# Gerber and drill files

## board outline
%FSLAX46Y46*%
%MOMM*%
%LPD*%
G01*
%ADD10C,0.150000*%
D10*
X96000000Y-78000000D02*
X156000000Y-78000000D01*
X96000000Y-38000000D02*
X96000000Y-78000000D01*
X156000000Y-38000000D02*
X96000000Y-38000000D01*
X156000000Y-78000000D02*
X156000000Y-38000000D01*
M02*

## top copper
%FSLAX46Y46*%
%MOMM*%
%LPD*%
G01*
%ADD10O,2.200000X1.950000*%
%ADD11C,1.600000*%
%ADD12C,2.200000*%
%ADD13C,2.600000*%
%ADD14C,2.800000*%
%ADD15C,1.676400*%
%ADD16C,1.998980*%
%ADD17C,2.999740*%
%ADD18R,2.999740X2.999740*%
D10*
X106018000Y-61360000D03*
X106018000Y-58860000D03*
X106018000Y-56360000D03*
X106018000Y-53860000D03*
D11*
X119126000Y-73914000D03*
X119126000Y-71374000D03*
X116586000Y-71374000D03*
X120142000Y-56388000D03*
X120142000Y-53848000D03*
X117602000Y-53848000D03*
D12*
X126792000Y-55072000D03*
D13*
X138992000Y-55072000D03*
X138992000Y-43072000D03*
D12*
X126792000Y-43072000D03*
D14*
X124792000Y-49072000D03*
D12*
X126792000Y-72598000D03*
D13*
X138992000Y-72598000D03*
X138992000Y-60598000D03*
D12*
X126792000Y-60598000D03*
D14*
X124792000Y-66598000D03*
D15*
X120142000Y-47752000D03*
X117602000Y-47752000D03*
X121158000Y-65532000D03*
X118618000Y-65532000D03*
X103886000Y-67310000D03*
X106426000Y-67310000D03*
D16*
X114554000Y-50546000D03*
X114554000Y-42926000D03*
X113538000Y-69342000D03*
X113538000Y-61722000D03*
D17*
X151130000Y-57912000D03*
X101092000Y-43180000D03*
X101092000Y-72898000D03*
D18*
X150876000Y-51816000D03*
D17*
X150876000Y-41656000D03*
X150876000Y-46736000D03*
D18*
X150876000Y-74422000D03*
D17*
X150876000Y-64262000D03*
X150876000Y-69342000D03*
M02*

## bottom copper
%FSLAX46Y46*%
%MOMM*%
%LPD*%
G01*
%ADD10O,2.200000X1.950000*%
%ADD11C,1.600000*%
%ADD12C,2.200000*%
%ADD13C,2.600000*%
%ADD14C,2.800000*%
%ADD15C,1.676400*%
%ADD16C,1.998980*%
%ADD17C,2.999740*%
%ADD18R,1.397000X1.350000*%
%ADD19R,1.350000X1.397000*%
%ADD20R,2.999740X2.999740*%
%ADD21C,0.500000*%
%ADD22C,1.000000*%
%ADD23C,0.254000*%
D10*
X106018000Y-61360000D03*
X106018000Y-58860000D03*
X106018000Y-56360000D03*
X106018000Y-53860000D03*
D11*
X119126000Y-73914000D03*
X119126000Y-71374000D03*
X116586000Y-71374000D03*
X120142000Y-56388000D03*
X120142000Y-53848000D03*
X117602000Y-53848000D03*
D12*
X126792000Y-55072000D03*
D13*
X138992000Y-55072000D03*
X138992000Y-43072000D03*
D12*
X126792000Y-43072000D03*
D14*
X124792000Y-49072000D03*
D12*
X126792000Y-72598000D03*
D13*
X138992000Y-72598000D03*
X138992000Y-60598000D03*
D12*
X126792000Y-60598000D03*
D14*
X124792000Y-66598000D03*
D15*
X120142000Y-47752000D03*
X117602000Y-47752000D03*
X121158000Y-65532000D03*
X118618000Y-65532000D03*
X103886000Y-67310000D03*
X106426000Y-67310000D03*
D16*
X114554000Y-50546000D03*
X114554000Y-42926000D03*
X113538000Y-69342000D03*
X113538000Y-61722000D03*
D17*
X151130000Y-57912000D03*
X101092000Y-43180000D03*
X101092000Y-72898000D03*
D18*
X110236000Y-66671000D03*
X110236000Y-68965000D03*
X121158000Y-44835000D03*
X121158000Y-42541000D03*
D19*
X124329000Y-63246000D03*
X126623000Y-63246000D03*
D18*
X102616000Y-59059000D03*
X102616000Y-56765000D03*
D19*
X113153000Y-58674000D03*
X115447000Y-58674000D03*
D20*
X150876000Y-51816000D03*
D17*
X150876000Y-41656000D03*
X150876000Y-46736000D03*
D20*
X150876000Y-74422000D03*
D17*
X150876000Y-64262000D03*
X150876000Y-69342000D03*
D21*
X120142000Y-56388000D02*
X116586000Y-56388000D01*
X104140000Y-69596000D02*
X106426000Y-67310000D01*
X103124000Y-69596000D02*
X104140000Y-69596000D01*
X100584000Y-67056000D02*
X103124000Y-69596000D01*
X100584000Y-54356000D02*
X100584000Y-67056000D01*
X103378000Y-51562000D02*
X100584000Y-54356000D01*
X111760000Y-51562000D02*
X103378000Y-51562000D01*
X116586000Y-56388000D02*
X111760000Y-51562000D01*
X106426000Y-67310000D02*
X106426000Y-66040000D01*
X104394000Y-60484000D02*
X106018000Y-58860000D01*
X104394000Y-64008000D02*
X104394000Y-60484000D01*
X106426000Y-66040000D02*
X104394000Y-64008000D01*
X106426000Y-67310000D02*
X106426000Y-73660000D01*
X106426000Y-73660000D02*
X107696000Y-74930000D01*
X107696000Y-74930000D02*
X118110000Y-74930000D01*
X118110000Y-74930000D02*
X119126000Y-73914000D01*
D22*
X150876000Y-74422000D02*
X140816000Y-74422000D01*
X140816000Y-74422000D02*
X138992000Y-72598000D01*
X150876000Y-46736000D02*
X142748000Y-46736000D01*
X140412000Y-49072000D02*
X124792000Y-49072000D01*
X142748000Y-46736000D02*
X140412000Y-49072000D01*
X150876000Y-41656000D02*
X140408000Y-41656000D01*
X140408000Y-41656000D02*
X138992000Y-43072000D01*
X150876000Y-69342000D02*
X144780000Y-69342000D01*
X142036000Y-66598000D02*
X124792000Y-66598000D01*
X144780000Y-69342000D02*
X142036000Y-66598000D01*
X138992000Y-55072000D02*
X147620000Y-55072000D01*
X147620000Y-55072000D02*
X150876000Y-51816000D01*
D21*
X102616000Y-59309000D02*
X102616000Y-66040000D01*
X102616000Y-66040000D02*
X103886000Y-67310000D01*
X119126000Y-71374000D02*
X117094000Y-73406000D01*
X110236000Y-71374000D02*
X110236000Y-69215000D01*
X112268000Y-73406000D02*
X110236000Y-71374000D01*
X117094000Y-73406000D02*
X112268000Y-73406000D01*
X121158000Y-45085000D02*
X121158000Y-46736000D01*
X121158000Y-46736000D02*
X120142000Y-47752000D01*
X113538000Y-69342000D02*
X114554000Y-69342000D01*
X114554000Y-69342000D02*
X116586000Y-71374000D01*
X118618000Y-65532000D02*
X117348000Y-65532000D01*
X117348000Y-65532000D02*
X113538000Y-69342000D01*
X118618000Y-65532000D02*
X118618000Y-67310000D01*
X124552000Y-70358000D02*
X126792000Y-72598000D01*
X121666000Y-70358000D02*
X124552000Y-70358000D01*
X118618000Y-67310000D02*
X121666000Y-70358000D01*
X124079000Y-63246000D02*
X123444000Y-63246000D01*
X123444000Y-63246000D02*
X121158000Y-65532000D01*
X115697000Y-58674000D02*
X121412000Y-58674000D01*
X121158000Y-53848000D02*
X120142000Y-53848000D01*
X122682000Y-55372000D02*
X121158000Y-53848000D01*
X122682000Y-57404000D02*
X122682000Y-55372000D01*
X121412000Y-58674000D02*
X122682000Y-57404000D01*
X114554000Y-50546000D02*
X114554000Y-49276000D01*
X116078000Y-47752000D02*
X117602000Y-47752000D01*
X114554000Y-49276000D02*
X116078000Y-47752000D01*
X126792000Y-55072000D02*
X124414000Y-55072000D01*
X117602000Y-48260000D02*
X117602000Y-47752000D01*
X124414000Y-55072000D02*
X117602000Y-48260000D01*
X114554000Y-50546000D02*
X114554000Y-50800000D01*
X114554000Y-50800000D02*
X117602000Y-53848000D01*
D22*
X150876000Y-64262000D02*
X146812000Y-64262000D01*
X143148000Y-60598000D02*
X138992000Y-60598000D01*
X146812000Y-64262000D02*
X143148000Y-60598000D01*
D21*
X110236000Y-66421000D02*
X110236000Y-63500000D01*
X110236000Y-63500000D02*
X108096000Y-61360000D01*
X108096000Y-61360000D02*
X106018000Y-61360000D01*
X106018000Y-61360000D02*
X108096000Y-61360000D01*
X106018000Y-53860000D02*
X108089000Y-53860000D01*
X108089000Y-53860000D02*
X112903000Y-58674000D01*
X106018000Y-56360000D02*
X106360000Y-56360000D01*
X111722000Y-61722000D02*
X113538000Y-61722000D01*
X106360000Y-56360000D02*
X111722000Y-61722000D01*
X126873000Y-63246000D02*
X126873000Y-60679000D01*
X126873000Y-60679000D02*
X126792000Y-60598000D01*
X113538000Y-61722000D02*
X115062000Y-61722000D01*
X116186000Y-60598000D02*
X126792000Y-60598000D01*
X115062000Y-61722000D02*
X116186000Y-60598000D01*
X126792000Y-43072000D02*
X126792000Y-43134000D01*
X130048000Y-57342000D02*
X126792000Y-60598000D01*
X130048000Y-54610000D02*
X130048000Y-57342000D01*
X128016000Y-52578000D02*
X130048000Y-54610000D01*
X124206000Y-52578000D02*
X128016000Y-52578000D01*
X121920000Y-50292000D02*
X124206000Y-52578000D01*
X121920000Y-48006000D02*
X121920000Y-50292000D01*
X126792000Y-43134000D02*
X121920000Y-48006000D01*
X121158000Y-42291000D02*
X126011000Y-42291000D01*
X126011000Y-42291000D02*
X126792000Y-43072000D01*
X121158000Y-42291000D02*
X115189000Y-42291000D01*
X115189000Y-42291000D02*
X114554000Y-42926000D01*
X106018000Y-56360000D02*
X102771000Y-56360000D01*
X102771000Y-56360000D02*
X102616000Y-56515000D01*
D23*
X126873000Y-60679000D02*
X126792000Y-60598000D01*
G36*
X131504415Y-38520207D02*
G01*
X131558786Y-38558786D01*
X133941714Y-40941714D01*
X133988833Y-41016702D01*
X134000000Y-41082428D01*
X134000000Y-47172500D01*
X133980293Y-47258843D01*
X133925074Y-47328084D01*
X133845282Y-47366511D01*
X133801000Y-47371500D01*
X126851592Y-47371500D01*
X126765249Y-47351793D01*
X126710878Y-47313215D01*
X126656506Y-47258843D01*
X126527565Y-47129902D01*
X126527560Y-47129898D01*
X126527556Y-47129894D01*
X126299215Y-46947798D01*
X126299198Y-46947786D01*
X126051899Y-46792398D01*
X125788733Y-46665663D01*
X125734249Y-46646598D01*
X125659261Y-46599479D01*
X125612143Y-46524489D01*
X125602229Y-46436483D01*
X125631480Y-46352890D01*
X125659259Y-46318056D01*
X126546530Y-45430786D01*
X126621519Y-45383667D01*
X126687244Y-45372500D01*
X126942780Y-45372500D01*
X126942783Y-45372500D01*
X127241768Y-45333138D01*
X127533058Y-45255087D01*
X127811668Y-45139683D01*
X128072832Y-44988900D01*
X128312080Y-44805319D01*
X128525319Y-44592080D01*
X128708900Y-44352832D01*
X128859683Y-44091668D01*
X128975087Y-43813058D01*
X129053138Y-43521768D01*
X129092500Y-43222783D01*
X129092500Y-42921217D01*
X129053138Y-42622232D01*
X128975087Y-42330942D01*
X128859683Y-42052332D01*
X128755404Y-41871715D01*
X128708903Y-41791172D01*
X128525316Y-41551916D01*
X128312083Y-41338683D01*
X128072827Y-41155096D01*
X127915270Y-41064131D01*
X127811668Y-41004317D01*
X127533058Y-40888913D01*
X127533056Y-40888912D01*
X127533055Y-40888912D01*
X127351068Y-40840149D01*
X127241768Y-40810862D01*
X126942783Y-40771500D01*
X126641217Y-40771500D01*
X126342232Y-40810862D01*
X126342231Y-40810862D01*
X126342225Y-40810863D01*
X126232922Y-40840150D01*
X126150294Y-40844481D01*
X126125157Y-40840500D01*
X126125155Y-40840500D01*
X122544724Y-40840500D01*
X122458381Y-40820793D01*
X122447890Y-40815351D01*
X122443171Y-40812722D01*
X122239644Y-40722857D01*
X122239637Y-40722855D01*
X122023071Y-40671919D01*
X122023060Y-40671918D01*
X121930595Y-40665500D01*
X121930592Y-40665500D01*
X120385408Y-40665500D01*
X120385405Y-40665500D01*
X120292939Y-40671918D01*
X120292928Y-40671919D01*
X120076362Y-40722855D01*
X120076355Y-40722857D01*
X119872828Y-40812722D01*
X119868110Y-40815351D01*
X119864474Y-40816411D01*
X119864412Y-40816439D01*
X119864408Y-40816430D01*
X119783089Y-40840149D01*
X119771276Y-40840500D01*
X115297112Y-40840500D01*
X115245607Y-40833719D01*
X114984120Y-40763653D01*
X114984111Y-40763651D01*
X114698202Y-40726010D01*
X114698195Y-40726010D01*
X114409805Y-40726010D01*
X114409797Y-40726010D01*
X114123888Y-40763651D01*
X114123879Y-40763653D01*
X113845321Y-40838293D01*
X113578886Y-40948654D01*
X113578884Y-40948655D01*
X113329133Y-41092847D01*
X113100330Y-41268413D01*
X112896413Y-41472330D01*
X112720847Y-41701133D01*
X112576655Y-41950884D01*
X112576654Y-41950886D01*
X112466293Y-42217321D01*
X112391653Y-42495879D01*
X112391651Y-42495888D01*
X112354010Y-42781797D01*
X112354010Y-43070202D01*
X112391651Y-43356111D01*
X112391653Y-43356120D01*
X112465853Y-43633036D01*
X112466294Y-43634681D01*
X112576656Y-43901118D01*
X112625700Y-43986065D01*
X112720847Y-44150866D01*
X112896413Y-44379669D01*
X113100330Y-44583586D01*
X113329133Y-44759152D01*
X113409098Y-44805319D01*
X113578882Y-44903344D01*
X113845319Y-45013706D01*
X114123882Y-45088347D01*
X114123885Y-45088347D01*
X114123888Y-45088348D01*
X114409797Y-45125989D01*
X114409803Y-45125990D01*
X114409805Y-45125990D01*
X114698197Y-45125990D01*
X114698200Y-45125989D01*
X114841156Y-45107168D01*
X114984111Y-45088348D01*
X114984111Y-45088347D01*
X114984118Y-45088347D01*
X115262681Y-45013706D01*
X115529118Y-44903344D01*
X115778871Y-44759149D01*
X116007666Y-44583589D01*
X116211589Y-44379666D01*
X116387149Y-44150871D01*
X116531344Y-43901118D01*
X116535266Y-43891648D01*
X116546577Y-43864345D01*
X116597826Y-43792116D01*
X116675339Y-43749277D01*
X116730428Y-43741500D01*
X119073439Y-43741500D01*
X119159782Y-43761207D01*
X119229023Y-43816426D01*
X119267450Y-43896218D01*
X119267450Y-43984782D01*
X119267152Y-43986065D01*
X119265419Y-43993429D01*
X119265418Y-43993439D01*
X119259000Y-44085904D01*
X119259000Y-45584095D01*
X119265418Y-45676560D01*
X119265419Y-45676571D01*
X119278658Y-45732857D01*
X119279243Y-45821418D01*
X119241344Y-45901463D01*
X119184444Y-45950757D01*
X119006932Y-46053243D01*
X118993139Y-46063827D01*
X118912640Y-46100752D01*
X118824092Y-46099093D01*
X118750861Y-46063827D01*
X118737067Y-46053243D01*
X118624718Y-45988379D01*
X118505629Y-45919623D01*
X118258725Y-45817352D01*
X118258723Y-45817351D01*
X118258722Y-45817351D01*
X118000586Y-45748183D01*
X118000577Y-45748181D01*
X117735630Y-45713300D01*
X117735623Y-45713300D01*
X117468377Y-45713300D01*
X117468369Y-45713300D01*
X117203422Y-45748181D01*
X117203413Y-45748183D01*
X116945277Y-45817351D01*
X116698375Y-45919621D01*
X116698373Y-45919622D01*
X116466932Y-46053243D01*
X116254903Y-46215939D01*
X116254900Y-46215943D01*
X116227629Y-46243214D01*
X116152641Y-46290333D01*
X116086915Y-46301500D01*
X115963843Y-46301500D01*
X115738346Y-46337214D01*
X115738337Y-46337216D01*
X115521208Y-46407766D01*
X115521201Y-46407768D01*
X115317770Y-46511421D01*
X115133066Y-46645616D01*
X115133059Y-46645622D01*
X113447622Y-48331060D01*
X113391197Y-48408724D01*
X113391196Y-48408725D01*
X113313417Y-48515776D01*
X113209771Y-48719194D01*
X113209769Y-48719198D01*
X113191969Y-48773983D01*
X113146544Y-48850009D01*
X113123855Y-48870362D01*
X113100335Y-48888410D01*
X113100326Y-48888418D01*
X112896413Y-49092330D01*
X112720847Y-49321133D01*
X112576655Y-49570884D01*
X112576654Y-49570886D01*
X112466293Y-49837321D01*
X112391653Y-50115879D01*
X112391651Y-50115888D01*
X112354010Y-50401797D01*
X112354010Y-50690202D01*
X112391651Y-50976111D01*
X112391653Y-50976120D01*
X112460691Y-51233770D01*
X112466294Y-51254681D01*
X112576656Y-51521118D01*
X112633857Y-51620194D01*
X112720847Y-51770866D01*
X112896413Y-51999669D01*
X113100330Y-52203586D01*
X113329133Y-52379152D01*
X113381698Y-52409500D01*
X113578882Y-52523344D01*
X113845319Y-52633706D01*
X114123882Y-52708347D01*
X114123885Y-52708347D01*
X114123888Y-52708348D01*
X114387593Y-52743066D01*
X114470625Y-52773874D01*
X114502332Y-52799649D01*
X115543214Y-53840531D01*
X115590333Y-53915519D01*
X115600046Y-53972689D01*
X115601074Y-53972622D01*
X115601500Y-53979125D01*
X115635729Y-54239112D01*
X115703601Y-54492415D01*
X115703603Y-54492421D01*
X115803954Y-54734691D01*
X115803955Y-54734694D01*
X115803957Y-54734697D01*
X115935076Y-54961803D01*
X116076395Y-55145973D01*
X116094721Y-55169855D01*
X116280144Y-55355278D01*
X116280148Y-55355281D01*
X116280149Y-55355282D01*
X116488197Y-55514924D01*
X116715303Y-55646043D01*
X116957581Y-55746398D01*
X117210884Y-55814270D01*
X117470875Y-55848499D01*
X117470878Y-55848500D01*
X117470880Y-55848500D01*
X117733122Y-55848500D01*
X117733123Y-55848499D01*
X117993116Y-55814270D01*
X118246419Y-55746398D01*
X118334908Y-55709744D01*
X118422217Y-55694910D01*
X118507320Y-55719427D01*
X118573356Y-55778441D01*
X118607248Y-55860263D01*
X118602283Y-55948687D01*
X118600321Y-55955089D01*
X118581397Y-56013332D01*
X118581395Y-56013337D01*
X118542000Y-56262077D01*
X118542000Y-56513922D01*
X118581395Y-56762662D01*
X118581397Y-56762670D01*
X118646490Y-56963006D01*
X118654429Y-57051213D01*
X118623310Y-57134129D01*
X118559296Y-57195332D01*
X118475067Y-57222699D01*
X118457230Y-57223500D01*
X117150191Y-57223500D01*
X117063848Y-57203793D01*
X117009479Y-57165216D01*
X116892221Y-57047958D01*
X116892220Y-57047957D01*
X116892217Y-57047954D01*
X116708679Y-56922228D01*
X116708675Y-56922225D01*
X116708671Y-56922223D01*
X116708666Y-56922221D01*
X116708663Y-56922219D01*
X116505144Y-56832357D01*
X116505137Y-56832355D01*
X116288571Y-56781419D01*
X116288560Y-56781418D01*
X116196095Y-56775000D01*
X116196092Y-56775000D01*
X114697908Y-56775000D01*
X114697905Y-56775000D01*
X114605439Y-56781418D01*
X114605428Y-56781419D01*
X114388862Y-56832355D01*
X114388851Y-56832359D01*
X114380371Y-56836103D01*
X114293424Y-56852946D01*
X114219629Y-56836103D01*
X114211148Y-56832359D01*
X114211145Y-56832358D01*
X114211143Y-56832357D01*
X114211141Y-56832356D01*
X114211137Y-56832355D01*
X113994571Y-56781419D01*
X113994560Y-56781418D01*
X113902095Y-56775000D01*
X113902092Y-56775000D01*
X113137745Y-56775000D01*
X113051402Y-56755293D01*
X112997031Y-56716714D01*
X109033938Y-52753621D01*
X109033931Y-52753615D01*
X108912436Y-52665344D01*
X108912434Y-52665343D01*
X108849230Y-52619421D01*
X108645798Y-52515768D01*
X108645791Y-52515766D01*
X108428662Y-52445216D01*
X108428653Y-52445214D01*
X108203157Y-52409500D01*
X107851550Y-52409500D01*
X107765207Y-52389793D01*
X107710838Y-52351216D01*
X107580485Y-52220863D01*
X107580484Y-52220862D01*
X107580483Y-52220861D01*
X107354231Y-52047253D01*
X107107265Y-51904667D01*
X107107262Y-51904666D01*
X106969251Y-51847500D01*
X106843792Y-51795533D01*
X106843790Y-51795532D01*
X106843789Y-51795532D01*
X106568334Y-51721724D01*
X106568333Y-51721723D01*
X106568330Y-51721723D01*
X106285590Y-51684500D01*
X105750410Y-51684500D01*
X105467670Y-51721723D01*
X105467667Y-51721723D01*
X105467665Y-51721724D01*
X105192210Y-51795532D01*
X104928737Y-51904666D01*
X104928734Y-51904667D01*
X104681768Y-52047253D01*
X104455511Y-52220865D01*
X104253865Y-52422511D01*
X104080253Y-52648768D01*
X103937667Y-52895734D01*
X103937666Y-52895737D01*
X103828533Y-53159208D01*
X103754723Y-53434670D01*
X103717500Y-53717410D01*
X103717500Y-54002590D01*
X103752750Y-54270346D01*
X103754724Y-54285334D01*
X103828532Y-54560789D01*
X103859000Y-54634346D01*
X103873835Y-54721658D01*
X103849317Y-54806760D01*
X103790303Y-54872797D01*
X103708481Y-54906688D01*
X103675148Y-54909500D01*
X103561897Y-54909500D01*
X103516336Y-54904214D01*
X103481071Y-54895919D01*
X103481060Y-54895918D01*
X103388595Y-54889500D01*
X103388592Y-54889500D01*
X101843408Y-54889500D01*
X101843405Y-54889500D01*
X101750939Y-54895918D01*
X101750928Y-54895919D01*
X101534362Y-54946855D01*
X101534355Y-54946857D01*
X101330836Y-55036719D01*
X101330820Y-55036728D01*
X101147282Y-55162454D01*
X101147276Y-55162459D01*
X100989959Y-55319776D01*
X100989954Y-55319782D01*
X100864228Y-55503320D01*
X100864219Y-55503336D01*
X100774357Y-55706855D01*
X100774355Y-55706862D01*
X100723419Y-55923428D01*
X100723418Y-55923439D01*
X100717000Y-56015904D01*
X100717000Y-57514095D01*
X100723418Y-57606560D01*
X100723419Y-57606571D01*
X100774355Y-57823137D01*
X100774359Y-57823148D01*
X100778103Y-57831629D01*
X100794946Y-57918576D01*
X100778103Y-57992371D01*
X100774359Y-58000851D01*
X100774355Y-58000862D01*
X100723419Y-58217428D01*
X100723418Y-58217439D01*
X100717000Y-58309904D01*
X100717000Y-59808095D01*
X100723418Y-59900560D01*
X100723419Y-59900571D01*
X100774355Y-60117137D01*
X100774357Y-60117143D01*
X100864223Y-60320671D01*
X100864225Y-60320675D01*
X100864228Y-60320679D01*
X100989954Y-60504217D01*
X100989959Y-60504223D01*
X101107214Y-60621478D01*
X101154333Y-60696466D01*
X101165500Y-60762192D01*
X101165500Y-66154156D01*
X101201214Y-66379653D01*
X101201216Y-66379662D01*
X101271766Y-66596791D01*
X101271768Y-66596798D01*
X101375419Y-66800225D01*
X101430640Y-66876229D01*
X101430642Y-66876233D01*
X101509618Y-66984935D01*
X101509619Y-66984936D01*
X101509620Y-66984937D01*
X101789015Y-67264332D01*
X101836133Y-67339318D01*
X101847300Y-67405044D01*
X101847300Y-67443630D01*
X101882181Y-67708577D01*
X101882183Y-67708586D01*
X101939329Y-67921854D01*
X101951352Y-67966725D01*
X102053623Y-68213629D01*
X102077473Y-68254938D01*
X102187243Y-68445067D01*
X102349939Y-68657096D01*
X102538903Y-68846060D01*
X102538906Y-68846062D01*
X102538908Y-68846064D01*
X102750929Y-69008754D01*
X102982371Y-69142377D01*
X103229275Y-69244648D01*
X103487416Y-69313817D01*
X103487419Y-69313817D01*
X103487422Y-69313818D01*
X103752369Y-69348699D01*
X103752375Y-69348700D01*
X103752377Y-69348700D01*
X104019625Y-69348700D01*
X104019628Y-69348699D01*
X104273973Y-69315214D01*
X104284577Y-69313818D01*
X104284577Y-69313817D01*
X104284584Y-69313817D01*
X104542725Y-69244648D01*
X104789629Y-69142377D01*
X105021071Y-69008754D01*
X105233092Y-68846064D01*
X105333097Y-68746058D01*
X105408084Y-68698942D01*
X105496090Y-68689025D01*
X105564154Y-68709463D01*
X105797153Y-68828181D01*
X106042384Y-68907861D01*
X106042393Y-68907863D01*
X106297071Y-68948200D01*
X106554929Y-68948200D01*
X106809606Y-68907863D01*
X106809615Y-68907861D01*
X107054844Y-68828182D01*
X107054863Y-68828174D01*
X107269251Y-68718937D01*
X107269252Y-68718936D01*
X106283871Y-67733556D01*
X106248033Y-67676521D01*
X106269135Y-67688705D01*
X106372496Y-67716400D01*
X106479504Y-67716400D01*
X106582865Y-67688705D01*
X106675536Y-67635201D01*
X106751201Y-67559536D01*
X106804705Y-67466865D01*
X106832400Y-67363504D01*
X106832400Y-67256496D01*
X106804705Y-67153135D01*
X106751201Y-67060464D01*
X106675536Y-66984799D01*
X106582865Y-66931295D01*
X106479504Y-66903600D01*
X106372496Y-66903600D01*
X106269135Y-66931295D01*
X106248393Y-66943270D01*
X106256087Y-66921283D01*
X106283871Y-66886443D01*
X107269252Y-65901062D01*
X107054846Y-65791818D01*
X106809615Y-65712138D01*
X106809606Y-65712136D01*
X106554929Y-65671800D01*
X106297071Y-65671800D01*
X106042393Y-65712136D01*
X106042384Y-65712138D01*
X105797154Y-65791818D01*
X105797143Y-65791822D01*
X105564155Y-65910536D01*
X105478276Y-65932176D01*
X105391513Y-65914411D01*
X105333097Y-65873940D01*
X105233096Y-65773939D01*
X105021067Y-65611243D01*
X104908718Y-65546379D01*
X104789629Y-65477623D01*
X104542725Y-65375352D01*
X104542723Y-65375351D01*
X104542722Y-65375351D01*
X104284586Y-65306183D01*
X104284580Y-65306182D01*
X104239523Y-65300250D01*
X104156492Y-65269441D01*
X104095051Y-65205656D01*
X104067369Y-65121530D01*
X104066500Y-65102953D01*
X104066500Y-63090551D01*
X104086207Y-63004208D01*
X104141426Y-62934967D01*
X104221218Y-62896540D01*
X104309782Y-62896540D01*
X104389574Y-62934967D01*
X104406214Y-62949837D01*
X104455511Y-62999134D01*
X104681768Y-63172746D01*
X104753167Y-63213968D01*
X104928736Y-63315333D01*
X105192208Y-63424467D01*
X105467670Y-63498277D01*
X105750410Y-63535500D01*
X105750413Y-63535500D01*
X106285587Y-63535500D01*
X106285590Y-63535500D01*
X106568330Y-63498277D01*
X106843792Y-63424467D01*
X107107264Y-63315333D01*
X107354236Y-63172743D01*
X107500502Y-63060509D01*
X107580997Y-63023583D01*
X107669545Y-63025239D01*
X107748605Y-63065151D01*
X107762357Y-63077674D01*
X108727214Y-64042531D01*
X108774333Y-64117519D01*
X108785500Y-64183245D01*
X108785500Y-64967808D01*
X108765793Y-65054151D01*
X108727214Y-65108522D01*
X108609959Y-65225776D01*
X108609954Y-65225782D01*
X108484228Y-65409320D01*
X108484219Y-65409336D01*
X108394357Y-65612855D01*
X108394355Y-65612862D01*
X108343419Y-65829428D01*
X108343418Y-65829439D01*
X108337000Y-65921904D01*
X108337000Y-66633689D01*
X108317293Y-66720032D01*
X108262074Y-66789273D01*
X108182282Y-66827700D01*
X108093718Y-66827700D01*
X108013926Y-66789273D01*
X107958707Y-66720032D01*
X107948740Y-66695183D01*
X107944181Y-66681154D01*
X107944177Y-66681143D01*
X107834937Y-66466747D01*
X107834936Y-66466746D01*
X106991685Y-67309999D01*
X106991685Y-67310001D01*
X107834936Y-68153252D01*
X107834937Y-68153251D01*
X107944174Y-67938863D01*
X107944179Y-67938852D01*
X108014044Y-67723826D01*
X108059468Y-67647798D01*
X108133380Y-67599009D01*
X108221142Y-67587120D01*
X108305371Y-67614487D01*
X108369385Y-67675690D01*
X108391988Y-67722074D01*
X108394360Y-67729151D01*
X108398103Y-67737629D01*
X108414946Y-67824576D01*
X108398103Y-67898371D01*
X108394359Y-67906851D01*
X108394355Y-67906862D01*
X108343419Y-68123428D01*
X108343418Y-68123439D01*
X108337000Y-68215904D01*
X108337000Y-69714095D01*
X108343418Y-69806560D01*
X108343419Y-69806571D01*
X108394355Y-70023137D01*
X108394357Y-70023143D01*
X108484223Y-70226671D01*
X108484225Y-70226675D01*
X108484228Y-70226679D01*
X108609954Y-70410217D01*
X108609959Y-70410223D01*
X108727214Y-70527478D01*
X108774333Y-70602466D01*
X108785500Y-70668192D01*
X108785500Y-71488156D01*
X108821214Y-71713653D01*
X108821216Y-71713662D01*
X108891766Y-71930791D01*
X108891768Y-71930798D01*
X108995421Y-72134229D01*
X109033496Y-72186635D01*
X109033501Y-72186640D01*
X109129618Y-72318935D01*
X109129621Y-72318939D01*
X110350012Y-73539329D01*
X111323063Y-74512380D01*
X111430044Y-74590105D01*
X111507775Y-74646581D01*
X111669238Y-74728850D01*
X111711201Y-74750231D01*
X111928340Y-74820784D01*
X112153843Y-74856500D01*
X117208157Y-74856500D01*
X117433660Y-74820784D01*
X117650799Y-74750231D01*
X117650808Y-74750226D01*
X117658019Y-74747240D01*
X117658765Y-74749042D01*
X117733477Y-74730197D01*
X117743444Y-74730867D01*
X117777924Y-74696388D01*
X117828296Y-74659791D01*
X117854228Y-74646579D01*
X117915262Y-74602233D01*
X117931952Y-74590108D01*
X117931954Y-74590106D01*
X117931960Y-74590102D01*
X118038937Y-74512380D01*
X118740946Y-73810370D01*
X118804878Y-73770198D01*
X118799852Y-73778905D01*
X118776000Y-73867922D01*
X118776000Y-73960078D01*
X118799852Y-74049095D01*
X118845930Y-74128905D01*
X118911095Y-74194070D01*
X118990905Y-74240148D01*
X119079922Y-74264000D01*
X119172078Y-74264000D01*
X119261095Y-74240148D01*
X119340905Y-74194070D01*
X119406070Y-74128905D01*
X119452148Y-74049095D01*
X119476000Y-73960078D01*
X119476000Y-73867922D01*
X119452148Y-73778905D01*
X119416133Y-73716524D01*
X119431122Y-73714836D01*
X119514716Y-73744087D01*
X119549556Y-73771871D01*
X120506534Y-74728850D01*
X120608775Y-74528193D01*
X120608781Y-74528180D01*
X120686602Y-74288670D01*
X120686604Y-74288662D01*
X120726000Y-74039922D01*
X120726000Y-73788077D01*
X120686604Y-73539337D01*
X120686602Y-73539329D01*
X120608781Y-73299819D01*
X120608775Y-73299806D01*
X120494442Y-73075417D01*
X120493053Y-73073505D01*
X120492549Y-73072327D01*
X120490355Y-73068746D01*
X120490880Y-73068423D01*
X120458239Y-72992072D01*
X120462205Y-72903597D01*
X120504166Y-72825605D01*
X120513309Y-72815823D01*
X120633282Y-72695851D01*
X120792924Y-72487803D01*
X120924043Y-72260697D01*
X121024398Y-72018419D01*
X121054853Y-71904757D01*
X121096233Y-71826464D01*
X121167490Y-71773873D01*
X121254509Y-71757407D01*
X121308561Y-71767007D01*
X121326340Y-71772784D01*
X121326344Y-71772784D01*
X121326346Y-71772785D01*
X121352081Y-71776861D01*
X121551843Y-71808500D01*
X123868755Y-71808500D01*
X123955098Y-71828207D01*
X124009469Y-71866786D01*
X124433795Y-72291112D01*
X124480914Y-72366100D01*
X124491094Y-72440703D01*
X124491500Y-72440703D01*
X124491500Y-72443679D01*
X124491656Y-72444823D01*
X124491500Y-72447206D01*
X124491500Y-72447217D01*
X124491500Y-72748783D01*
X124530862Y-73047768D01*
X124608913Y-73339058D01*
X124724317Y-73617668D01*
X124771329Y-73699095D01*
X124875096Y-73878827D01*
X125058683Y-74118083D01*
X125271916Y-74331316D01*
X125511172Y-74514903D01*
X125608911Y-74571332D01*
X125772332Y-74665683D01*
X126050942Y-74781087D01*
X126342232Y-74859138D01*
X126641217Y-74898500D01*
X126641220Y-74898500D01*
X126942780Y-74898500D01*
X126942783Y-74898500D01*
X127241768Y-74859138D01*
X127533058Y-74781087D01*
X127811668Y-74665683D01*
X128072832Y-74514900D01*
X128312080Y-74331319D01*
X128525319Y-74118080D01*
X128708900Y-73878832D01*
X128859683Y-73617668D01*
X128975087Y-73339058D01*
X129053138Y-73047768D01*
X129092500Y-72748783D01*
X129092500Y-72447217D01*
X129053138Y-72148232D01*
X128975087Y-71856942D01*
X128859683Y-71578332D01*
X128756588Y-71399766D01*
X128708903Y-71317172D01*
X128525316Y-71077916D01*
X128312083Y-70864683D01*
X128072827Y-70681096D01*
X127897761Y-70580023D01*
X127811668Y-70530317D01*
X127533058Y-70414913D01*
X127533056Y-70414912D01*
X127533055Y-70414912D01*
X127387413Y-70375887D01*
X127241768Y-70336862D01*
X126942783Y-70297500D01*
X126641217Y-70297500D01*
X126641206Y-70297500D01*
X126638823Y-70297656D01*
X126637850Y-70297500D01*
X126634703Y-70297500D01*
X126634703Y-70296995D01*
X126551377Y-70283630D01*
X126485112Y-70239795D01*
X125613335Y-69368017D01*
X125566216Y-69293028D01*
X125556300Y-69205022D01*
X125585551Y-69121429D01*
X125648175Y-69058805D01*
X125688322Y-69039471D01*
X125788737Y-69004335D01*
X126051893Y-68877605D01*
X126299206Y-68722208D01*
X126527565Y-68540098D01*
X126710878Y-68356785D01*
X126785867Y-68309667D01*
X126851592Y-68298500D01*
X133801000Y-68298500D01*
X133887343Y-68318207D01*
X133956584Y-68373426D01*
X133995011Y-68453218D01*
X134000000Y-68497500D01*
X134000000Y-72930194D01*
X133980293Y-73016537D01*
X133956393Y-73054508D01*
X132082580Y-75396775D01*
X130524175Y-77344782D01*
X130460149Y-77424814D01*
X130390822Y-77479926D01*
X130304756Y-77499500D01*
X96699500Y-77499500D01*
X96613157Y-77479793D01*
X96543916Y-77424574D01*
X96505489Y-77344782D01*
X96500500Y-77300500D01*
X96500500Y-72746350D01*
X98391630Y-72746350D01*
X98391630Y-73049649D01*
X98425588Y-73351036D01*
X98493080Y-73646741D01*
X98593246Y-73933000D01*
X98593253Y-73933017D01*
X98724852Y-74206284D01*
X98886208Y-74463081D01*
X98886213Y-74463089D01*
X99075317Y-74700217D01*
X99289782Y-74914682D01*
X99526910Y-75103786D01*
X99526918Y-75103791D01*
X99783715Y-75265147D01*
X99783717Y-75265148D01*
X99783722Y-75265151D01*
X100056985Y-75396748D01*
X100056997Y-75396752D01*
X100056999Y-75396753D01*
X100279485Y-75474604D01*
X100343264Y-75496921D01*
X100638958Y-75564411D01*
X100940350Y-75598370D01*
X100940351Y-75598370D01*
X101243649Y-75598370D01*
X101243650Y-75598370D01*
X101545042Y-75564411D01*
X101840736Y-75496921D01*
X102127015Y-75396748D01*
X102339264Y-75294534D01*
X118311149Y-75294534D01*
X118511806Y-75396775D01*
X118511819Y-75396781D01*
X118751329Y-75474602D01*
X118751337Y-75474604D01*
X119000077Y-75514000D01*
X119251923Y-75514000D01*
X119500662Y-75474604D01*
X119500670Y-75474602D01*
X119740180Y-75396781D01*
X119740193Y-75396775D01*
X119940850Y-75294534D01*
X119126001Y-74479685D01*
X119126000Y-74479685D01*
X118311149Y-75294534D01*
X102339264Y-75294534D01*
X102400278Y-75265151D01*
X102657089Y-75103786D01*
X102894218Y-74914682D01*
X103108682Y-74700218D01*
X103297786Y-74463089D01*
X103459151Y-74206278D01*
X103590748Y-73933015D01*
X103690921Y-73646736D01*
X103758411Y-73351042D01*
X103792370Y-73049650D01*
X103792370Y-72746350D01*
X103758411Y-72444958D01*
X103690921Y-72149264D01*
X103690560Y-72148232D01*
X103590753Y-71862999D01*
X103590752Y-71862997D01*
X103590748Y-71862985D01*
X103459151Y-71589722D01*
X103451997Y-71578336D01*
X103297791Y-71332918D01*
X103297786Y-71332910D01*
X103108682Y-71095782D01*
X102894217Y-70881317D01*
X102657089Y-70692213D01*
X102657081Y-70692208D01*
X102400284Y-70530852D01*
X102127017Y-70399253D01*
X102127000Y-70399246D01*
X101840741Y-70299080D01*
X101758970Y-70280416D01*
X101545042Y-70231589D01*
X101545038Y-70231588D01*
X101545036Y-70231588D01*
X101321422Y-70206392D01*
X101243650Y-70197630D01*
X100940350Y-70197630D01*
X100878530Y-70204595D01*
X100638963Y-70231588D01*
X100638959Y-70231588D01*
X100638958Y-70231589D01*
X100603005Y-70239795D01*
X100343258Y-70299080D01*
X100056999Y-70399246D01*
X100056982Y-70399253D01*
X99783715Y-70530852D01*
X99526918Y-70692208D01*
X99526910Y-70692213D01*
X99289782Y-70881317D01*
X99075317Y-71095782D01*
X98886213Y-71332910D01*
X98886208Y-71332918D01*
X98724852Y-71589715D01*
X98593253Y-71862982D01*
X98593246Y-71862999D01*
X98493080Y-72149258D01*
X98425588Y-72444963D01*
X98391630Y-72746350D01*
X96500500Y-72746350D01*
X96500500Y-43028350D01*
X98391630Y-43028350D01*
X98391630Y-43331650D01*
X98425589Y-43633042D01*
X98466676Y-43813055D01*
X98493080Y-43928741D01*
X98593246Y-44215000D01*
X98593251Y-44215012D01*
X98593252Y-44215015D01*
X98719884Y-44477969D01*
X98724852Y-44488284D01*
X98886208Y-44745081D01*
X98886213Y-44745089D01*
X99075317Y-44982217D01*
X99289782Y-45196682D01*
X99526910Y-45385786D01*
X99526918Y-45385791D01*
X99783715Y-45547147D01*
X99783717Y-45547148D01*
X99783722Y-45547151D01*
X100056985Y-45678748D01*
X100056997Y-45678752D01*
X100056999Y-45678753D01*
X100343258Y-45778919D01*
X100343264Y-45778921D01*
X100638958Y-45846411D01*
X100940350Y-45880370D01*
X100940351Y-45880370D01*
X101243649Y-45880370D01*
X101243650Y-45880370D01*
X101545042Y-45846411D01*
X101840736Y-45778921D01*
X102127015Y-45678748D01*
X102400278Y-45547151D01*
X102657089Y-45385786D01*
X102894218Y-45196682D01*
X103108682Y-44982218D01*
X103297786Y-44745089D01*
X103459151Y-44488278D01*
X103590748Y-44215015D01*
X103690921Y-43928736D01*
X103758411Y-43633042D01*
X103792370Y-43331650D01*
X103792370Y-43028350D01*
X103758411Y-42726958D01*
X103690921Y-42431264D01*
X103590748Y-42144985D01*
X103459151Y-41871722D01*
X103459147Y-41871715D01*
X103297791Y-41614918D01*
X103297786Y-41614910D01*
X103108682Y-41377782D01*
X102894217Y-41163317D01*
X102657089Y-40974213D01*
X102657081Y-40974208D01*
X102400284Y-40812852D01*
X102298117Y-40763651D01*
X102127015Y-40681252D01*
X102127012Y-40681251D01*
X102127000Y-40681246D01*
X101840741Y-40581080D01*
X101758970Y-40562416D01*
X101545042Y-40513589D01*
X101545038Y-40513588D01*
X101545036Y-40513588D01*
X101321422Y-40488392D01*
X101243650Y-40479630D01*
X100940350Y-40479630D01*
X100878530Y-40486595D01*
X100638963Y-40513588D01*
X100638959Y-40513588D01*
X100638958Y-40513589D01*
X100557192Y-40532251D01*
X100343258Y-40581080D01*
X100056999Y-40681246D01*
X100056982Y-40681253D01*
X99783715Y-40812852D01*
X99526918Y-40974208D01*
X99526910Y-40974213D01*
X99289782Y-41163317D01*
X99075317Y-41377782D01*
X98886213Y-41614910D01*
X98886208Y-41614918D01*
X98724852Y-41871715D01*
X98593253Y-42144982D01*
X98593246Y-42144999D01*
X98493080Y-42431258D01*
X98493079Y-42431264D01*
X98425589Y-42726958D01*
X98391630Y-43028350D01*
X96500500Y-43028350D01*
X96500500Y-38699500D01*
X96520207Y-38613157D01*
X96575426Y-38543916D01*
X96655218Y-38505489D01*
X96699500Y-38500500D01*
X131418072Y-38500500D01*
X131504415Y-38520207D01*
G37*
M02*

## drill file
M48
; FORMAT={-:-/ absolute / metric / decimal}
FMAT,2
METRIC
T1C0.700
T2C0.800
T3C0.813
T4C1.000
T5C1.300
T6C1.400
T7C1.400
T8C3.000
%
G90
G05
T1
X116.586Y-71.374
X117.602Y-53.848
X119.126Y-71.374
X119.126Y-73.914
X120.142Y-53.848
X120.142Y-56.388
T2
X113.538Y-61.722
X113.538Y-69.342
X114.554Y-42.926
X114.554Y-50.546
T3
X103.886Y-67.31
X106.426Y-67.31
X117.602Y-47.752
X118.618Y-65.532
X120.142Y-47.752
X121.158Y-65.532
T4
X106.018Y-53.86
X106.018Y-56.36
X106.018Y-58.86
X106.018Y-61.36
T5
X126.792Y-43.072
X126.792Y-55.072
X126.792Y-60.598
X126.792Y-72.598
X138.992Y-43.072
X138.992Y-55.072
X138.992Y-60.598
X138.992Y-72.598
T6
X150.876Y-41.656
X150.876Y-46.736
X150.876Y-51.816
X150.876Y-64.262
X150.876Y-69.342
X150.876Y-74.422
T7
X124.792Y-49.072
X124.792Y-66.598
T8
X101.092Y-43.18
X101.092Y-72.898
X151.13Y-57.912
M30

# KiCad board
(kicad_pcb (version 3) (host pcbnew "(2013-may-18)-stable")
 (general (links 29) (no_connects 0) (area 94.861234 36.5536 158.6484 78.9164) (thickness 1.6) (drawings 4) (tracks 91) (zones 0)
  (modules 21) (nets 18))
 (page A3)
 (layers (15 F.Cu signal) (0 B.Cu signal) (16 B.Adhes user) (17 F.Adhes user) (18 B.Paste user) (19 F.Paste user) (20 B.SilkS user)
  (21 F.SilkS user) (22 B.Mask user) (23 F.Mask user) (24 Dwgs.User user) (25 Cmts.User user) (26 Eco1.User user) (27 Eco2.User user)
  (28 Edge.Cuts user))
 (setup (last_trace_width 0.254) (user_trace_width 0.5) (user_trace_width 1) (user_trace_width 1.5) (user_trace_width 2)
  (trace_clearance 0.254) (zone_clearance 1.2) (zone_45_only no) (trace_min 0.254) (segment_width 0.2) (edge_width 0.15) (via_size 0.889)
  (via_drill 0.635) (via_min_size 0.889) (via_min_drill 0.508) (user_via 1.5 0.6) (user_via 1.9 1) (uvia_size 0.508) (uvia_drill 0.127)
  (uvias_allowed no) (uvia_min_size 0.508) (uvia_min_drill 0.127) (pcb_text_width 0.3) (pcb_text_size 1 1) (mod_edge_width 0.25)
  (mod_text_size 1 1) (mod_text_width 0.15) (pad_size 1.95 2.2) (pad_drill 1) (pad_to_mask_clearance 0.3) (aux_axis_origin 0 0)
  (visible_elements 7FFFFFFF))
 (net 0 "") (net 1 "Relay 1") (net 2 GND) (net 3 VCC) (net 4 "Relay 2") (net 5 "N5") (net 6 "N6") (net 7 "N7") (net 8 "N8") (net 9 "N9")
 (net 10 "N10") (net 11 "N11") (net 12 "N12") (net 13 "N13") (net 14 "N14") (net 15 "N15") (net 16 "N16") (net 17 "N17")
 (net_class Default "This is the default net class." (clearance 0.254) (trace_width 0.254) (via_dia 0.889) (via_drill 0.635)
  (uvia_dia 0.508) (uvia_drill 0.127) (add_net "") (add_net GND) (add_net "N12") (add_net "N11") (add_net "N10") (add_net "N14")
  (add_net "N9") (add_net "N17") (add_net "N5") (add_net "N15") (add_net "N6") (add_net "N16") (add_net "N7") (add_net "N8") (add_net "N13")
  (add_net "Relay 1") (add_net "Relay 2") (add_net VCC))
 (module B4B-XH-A (layer F.Cu) (at 106.018 57.61 90)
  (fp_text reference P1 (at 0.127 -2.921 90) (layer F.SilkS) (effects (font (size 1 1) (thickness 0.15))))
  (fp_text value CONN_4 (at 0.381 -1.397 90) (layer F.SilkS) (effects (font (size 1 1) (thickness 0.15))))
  (pad 1 thru_hole oval (at -3.75 0 90) (size 1.95 2.2) (drill 1) (layers *.Cu *.Mask F.SilkS) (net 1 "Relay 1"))
  (pad 2 thru_hole oval (at -1.25 0 90) (size 1.95 2.2) (drill 1) (layers *.Cu *.Mask F.SilkS) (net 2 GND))
  (pad 3 thru_hole oval (at 1.25 0 90) (size 1.95 2.2) (drill 1) (layers *.Cu *.Mask F.SilkS) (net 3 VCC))
  (pad 4 thru_hole oval (at 3.75 0 90) (size 1.95 2.2) (drill 1) (layers *.Cu *.Mask F.SilkS) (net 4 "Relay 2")))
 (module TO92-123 (layer F.Cu) (at 117.856 72.644 270)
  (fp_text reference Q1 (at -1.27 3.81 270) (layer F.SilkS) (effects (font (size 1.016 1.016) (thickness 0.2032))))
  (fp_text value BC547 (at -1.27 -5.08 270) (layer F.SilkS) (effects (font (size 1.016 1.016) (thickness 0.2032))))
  (pad 3 thru_hole circle (at 1.27 -1.27 270) (size 1.6 1.6) (drill 0.7) (layers *.Cu *.Mask F.SilkS) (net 2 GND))
  (pad 2 thru_hole circle (at -1.27 -1.27 270) (size 1.6 1.6) (drill 0.7) (layers *.Cu *.Mask F.SilkS) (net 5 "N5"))
  (pad 1 thru_hole circle (at -1.27 1.27 270) (size 1.6 1.6) (drill 0.7) (layers *.Cu *.Mask F.SilkS) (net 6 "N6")))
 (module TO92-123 (layer F.Cu) (at 118.872 55.118 270)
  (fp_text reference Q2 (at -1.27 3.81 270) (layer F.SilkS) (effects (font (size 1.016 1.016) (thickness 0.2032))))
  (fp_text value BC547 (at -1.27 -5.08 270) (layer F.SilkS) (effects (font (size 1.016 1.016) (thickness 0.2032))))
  (pad 3 thru_hole circle (at 1.27 -1.27 270) (size 1.6 1.6) (drill 0.7) (layers *.Cu *.Mask F.SilkS) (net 2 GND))
  (pad 2 thru_hole circle (at -1.27 -1.27 270) (size 1.6 1.6) (drill 0.7) (layers *.Cu *.Mask F.SilkS) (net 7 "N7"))
  (pad 1 thru_hole circle (at -1.27 1.27 270) (size 1.6 1.6) (drill 0.7) (layers *.Cu *.Mask F.SilkS) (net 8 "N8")))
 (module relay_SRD (layer F.Cu) (at 132.842 49.022)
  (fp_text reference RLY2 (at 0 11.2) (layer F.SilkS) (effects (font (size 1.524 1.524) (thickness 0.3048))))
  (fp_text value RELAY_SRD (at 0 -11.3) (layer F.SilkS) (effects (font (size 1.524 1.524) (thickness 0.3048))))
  (pad 2 thru_hole circle (at -6.05 6.05 90) (size 2.2 2.2) (drill 1.3) (layers *.Cu *.Mask) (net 8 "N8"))
  (pad 3 thru_hole circle (at 6.15 6.05 90) (size 2.6 2.6) (drill 1.3) (layers *.Cu *.Mask) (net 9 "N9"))
  (pad 4 thru_hole circle (at 6.15 -5.95 90) (size 2.6 2.6) (drill 1.3) (layers *.Cu *.Mask) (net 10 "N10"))
  (pad 5 thru_hole circle (at -6.05 -5.95 90) (size 2.2 2.2) (drill 1.3) (layers *.Cu *.Mask F.SilkS) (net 3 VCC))
  (pad 1 thru_hole circle (at -8.05 0.05 90) (size 2.8 2.8) (drill 1.4) (layers *.Cu *.Mask) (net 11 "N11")))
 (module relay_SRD (layer F.Cu) (at 132.842 66.548)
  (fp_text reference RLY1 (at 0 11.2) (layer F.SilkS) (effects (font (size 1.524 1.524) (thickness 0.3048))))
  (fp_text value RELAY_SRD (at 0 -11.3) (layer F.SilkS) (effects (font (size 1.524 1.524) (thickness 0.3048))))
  (pad 2 thru_hole circle (at -6.05 6.05 90) (size 2.2 2.2) (drill 1.3) (layers *.Cu *.Mask) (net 6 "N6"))
  (pad 3 thru_hole circle (at 6.15 6.05 90) (size 2.6 2.6) (drill 1.3) (layers *.Cu *.Mask) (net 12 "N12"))
  (pad 4 thru_hole circle (at 6.15 -5.95 90) (size 2.6 2.6) (drill 1.3) (layers *.Cu *.Mask) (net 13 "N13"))
  (pad 5 thru_hole circle (at -6.05 -5.95 90) (size 2.2 2.2) (drill 1.3) (layers *.Cu *.Mask F.SilkS) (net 3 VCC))
  (pad 1 thru_hole circle (at -8.05 0.05 90) (size 2.8 2.8) (drill 1.4) (layers *.Cu *.Mask) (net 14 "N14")))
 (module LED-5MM (layer F.Cu) (at 118.872 47.752 180)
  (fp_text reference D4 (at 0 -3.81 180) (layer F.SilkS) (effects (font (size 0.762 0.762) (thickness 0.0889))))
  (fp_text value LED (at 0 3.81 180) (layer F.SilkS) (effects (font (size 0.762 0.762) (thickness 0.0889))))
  (pad 1 thru_hole circle (at -1.27 0 180) (size 1.6764 1.6764) (drill 0.8128) (layers *.Cu *.Mask F.SilkS) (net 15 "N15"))
  (pad 2 thru_hole circle (at 1.27 0 180) (size 1.6764 1.6764) (drill 0.8128) (layers *.Cu *.Mask F.SilkS) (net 8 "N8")))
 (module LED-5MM (layer F.Cu) (at 119.888 65.532 180)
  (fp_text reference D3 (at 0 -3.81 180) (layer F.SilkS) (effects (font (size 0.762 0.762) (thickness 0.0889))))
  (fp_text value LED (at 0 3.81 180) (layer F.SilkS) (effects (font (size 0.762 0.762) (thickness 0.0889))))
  (pad 1 thru_hole circle (at -1.27 0 180) (size 1.6764 1.6764) (drill 0.8128) (layers *.Cu *.Mask F.SilkS) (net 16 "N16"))
  (pad 2 thru_hole circle (at 1.27 0 180) (size 1.6764 1.6764) (drill 0.8128) (layers *.Cu *.Mask F.SilkS) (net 6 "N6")))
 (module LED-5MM (layer F.Cu) (at 105.156 67.31)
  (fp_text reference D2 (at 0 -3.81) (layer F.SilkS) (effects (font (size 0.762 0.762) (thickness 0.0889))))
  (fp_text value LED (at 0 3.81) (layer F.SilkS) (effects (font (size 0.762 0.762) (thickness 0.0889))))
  (pad 1 thru_hole circle (at -1.27 0) (size 1.6764 1.6764) (drill 0.8128) (layers *.Cu *.Mask F.SilkS) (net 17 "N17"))
  (pad 2 thru_hole circle (at 1.27 0) (size 1.6764 1.6764) (drill 0.8128) (layers *.Cu *.Mask F.SilkS) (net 2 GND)))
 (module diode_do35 (layer F.Cu) (at 114.554 46.736 90)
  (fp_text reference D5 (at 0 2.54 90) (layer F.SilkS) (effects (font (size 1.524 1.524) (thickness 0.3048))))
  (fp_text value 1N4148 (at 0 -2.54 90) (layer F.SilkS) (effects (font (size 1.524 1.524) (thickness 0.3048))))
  (pad 1 thru_hole circle (at -3.81 0 90) (size 1.99898 1.99898) (drill 0.8001) (layers *.Cu *.Mask F.SilkS) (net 8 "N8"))
  (pad 2 thru_hole circle (at 3.81 0 90) (size 1.99898 1.99898) (drill 0.8001) (layers *.Cu *.Mask F.SilkS) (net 3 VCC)))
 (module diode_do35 (layer F.Cu) (at 113.538 65.532 90)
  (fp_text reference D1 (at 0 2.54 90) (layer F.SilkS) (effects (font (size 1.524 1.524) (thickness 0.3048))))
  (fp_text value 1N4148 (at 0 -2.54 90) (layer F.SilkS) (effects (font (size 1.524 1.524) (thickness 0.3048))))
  (pad 1 thru_hole circle (at -3.81 0 90) (size 1.99898 1.99898) (drill 0.8001) (layers *.Cu *.Mask F.SilkS) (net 6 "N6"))
  (pad 2 thru_hole circle (at 3.81 0 90) (size 1.99898 1.99898) (drill 0.8001) (layers *.Cu *.Mask F.SilkS) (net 3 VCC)))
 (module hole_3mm (layer F.Cu) (at 151.13 57.912)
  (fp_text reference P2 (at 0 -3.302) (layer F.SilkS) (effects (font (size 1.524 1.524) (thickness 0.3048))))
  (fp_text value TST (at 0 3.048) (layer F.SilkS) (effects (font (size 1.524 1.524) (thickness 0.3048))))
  (pad 1 thru_hole circle (at 0 0) (size 2.99974 2.99974) (drill 2.99974) (layers *.Cu F.SilkS)))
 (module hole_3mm (layer F.Cu) (at 101.092 43.18)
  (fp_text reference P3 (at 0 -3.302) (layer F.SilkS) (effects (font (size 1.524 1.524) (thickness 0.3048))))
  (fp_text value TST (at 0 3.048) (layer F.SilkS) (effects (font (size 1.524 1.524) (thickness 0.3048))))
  (pad 1 thru_hole circle (at 0 0) (size 2.99974 2.99974) (drill 2.99974) (layers *.Cu F.SilkS)))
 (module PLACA (layer F.Cu) (at 96 78)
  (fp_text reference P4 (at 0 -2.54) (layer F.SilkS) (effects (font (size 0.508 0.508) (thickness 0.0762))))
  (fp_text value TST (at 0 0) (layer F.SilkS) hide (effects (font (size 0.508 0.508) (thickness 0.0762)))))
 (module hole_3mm (layer F.Cu) (at 101.092 72.898)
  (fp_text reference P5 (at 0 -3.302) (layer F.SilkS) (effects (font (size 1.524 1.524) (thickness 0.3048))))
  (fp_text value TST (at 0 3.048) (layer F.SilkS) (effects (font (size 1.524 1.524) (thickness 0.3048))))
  (pad 1 thru_hole circle (at 0 0) (size 2.99974 2.99974) (drill 2.99974) (layers *.Cu F.SilkS)))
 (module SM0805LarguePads (layer B.Cu) (at 110.236 67.818 270)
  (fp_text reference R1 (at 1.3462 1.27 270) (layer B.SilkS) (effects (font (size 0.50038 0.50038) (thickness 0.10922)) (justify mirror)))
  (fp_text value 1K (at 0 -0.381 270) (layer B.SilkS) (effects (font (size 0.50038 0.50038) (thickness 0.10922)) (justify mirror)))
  (pad 1 smd rect (at -1.147 0 270) (size 1.35 1.397) (layers B.Cu B.Paste B.Mask) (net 1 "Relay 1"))
  (pad 2 smd rect (at 1.147 0 270) (size 1.35 1.397) (layers B.Cu B.Paste B.Mask) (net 5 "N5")))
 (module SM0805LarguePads (layer B.Cu) (at 121.158 43.688 90)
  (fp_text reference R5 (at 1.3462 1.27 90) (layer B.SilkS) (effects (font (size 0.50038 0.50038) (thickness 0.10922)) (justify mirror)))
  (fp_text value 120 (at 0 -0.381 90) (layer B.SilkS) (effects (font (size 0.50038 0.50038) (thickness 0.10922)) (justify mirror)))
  (pad 1 smd rect (at -1.147 0 90) (size 1.35 1.397) (layers B.Cu B.Paste B.Mask) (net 15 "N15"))
  (pad 2 smd rect (at 1.147 0 90) (size 1.35 1.397) (layers B.Cu B.Paste B.Mask) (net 3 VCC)))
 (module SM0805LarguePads (layer B.Cu) (at 125.476 63.246)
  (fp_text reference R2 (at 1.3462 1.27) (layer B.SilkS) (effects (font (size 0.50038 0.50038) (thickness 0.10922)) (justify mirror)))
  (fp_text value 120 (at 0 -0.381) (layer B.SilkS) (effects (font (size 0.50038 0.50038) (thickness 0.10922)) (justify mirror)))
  (pad 1 smd rect (at -1.147 0) (size 1.35 1.397) (layers B.Cu B.Paste B.Mask) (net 16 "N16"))
  (pad 2 smd rect (at 1.147 0) (size 1.35 1.397) (layers B.Cu B.Paste B.Mask) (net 3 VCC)))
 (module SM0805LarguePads (layer B.Cu) (at 102.616 57.912 90)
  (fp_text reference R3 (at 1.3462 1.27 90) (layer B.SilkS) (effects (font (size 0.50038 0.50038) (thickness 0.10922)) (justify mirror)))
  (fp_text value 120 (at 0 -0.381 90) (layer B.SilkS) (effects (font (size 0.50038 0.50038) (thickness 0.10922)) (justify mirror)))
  (pad 1 smd rect (at -1.147 0 90) (size 1.35 1.397) (layers B.Cu B.Paste B.Mask) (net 17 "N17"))
  (pad 2 smd rect (at 1.147 0 90) (size 1.35 1.397) (layers B.Cu B.Paste B.Mask) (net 3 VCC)))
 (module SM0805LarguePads (layer B.Cu) (at 114.3 58.674)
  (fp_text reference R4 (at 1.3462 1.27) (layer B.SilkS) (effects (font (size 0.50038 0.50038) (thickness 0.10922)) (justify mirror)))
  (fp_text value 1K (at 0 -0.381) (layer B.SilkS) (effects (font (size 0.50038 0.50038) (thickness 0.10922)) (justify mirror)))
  (pad 1 smd rect (at -1.147 0) (size 1.35 1.397) (layers B.Cu B.Paste B.Mask) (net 4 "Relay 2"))
  (pad 2 smd rect (at 1.147 0) (size 1.35 1.397) (layers B.Cu B.Paste B.Mask) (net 7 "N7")))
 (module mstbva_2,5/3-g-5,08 (layer F.Cu) (at 150.876 46.736 90)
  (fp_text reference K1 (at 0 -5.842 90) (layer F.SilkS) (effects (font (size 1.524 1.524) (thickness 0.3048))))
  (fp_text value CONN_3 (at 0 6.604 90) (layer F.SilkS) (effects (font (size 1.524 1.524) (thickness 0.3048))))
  (pad 1 thru_hole rect (at -5.08 0 90) (size 2.99974 2.99974) (drill 1.39954) (layers *.Cu *.Mask F.SilkS) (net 9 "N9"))
  (pad 3 thru_hole circle (at 5.08 0 90) (size 2.99974 2.99974) (drill 1.39954) (layers *.Cu *.Mask F.SilkS) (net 10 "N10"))
  (pad 2 thru_hole circle (at 0 0 90) (size 2.99974 2.99974) (drill 1.39954) (layers *.Cu *.Mask F.SilkS) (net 11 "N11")))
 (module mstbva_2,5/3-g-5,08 (layer F.Cu) (at 150.876 69.342 90)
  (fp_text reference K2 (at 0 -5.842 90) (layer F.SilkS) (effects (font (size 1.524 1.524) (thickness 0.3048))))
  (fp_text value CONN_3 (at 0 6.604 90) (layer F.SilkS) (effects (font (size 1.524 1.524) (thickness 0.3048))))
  (pad 1 thru_hole rect (at -5.08 0 90) (size 2.99974 2.99974) (drill 1.39954) (layers *.Cu *.Mask F.SilkS) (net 12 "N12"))
  (pad 3 thru_hole circle (at 5.08 0 90) (size 2.99974 2.99974) (drill 1.39954) (layers *.Cu *.Mask F.SilkS) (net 13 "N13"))
  (pad 2 thru_hole circle (at 0 0 90) (size 2.99974 2.99974) (drill 1.39954) (layers *.Cu *.Mask F.SilkS) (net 14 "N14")))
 (gr_line (start 96 78) (end 156 78) (angle 90) (layer Edge.Cuts) (width 0.15))
 (gr_line (start 96 38) (end 96 78) (angle 90) (layer Edge.Cuts) (width 0.15))
 (gr_line (start 156 38) (end 96 38) (angle 90) (layer Edge.Cuts) (width 0.15))
 (gr_line (start 156 78) (end 156 38) (angle 90) (layer Edge.Cuts) (width 0.15))
 (segment (start 120.142 56.388) (end 116.586 56.388) (width 0.5) (layer B.Cu) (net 2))
 (segment (start 104.14 69.596) (end 106.426 67.31) (width 0.5) (layer B.Cu) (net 2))
 (segment (start 103.124 69.596) (end 104.14 69.596) (width 0.5) (layer B.Cu) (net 2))
 (segment (start 100.584 67.056) (end 103.124 69.596) (width 0.5) (layer B.Cu) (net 2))
 (segment (start 100.584 54.356) (end 100.584 67.056) (width 0.5) (layer B.Cu) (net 2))
 (segment (start 103.378 51.562) (end 100.584 54.356) (width 0.5) (layer B.Cu) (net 2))
 (segment (start 111.76 51.562) (end 103.378 51.562) (width 0.5) (layer B.Cu) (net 2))
 (segment (start 116.586 56.388) (end 111.76 51.562) (width 0.5) (layer B.Cu) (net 2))
 (segment (start 106.426 67.31) (end 106.426 66.04) (width 0.5) (layer B.Cu) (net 2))
 (segment (start 104.394 60.484) (end 106.018 58.86) (width 0.5) (layer B.Cu) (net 2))
 (segment (start 104.394 64.008) (end 104.394 60.484) (width 0.5) (layer B.Cu) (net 2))
 (segment (start 106.426 66.04) (end 104.394 64.008) (width 0.5) (layer B.Cu) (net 2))
 (segment (start 106.426 67.31) (end 106.426 73.66) (width 0.5) (layer B.Cu) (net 2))
 (segment (start 106.426 73.66) (end 107.696 74.93) (width 0.5) (layer B.Cu) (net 2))
 (segment (start 107.696 74.93) (end 118.11 74.93) (width 0.5) (layer B.Cu) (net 2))
 (segment (start 118.11 74.93) (end 119.126 73.914) (width 0.5) (layer B.Cu) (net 2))
 (segment (start 150.876 74.422) (end 140.816 74.422) (width 1) (layer B.Cu) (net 12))
 (segment (start 140.816 74.422) (end 138.992 72.598) (width 1) (layer B.Cu) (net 12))
 (segment (start 150.876 46.736) (end 142.748 46.736) (width 1) (layer B.Cu) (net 11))
 (segment (start 140.412 49.072) (end 124.792 49.072) (width 1) (layer B.Cu) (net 11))
 (segment (start 142.748 46.736) (end 140.412 49.072) (width 1) (layer B.Cu) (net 11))
 (segment (start 150.876 41.656) (end 140.408 41.656) (width 1) (layer B.Cu) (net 10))
 (segment (start 140.408 41.656) (end 138.992 43.072) (width 1) (layer B.Cu) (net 10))
 (segment (start 150.876 69.342) (end 144.78 69.342) (width 1) (layer B.Cu) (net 14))
 (segment (start 142.036 66.598) (end 124.792 66.598) (width 1) (layer B.Cu) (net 14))
 (segment (start 144.78 69.342) (end 142.036 66.598) (width 1) (layer B.Cu) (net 14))
 (segment (start 138.992 55.072) (end 147.62 55.072) (width 1) (layer B.Cu) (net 9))
 (segment (start 147.62 55.072) (end 150.876 51.816) (width 1) (layer B.Cu) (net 9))
 (segment (start 102.616 59.309) (end 102.616 66.04) (width 0.5) (layer B.Cu) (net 17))
 (segment (start 102.616 66.04) (end 103.886 67.31) (width 0.5) (layer B.Cu) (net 17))
 (segment (start 119.126 71.374) (end 117.094 73.406) (width 0.5) (layer B.Cu) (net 5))
 (segment (start 110.236 71.374) (end 110.236 69.215) (width 0.5) (layer B.Cu) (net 5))
 (segment (start 112.268 73.406) (end 110.236 71.374) (width 0.5) (layer B.Cu) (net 5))
 (segment (start 117.094 73.406) (end 112.268 73.406) (width 0.5) (layer B.Cu) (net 5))
 (segment (start 121.158 45.085) (end 121.158 46.736) (width 0.5) (layer B.Cu) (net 15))
 (segment (start 121.158 46.736) (end 120.142 47.752) (width 0.5) (layer B.Cu) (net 15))
 (segment (start 113.538 69.342) (end 114.554 69.342) (width 0.5) (layer B.Cu) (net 6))
 (segment (start 114.554 69.342) (end 116.586 71.374) (width 0.5) (layer B.Cu) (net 6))
 (segment (start 118.618 65.532) (end 117.348 65.532) (width 0.5) (layer B.Cu) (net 6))
 (segment (start 117.348 65.532) (end 113.538 69.342) (width 0.5) (layer B.Cu) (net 6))
 (segment (start 118.618 65.532) (end 118.618 67.31) (width 0.5) (layer B.Cu) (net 6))
 (segment (start 124.552 70.358) (end 126.792 72.598) (width 0.5) (layer B.Cu) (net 6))
 (segment (start 121.666 70.358) (end 124.552 70.358) (width 0.5) (layer B.Cu) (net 6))
 (segment (start 118.618 67.31) (end 121.666 70.358) (width 0.5) (layer B.Cu) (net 6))
 (segment (start 124.079 63.246) (end 123.444 63.246) (width 0.5) (layer B.Cu) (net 16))
 (segment (start 123.444 63.246) (end 121.158 65.532) (width 0.5) (layer B.Cu) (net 16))
 (segment (start 115.697 58.674) (end 121.412 58.674) (width 0.5) (layer B.Cu) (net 7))
 (segment (start 121.158 53.848) (end 120.142 53.848) (width 0.5) (layer B.Cu) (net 7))
 (segment (start 122.682 55.372) (end 121.158 53.848) (width 0.5) (layer B.Cu) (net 7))
 (segment (start 122.682 57.404) (end 122.682 55.372) (width 0.5) (layer B.Cu) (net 7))
 (segment (start 121.412 58.674) (end 122.682 57.404) (width 0.5) (layer B.Cu) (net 7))
 (segment (start 114.554 50.546) (end 114.554 49.276) (width 0.5) (layer B.Cu) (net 8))
 (segment (start 116.078 47.752) (end 117.602 47.752) (width 0.5) (layer B.Cu) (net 8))
 (segment (start 114.554 49.276) (end 116.078 47.752) (width 0.5) (layer B.Cu) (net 8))
 (segment (start 126.792 55.072) (end 124.414 55.072) (width 0.5) (layer B.Cu) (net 8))
 (segment (start 117.602 48.26) (end 117.602 47.752) (width 0.5) (layer B.Cu) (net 8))
 (segment (start 124.414 55.072) (end 117.602 48.26) (width 0.5) (layer B.Cu) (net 8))
 (segment (start 114.554 50.546) (end 114.554 50.8) (width 0.5) (layer B.Cu) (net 8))
 (segment (start 114.554 50.8) (end 117.602 53.848) (width 0.5) (layer B.Cu) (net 8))
 (segment (start 150.876 64.262) (end 146.812 64.262) (width 1) (layer B.Cu) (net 13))
 (segment (start 143.148 60.598) (end 138.992 60.598) (width 1) (layer B.Cu) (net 13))
 (segment (start 146.812 64.262) (end 143.148 60.598) (width 1) (layer B.Cu) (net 13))
 (segment (start 110.236 66.421) (end 110.236 63.5) (width 0.5) (layer B.Cu) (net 1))
 (segment (start 110.236 63.5) (end 108.096 61.36) (width 0.5) (layer B.Cu) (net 1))
 (segment (start 108.096 61.36) (end 106.018 61.36) (width 0.5) (layer B.Cu) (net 1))
 (segment (start 106.018 61.36) (end 108.096 61.36) (width 0.5) (layer B.Cu) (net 1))
 (segment (start 106.018 53.86) (end 108.089 53.86) (width 0.5) (layer B.Cu) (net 4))
 (segment (start 108.089 53.86) (end 112.903 58.674) (width 0.5) (layer B.Cu) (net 4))
 (segment (start 106.018 56.36) (end 106.36 56.36) (width 0.5) (layer B.Cu) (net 3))
 (segment (start 111.722 61.722) (end 113.538 61.722) (width 0.5) (layer B.Cu) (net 3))
 (segment (start 106.36 56.36) (end 111.722 61.722) (width 0.5) (layer B.Cu) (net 3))
 (segment (start 126.873 63.246) (end 126.873 60.679) (width 0.5) (layer B.Cu) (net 3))
 (segment (start 126.873 60.679) (end 126.792 60.598) (width 0.5) (layer B.Cu) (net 3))
 (segment (start 113.538 61.722) (end 115.062 61.722) (width 0.5) (layer B.Cu) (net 3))
 (segment (start 116.186 60.598) (end 126.792 60.598) (width 0.5) (layer B.Cu) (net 3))
 (segment (start 115.062 61.722) (end 116.186 60.598) (width 0.5) (layer B.Cu) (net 3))
 (segment (start 126.792 43.072) (end 126.792 43.134) (width 0.5) (layer B.Cu) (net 3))
 (segment (start 130.048 57.342) (end 126.792 60.598) (width 0.5) (layer B.Cu) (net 3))
 (segment (start 130.048 54.61) (end 130.048 57.342) (width 0.5) (layer B.Cu) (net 3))
 (segment (start 128.016 52.578) (end 130.048 54.61) (width 0.5) (layer B.Cu) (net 3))
 (segment (start 124.206 52.578) (end 128.016 52.578) (width 0.5) (layer B.Cu) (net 3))
 (segment (start 121.92 50.292) (end 124.206 52.578) (width 0.5) (layer B.Cu) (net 3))
 (segment (start 121.92 48.006) (end 121.92 50.292) (width 0.5) (layer B.Cu) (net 3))
 (segment (start 126.792 43.134) (end 121.92 48.006) (width 0.5) (layer B.Cu) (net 3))
 (segment (start 121.158 42.291) (end 126.011 42.291) (width 0.5) (layer B.Cu) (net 3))
 (segment (start 126.011 42.291) (end 126.792 43.072) (width 0.5) (layer B.Cu) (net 3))
 (segment (start 121.158 42.291) (end 115.189 42.291) (width 0.5) (layer B.Cu) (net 3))
 (segment (start 115.189 42.291) (end 114.554 42.926) (width 0.5) (layer B.Cu) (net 3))
 (segment (start 106.018 56.36) (end 102.771 56.36) (width 0.5) (layer B.Cu) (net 3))
 (segment (start 102.771 56.36) (end 102.616 56.515) (width 0.5) (layer B.Cu) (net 3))
 (segment (start 126.873 60.679) (end 126.792 60.598) (width 0.254) (layer B.Cu) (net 3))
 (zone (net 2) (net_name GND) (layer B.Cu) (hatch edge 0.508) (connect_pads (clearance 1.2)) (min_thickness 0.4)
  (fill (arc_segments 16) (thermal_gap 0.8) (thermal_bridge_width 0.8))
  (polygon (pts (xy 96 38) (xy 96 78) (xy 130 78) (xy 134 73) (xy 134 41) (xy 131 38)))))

